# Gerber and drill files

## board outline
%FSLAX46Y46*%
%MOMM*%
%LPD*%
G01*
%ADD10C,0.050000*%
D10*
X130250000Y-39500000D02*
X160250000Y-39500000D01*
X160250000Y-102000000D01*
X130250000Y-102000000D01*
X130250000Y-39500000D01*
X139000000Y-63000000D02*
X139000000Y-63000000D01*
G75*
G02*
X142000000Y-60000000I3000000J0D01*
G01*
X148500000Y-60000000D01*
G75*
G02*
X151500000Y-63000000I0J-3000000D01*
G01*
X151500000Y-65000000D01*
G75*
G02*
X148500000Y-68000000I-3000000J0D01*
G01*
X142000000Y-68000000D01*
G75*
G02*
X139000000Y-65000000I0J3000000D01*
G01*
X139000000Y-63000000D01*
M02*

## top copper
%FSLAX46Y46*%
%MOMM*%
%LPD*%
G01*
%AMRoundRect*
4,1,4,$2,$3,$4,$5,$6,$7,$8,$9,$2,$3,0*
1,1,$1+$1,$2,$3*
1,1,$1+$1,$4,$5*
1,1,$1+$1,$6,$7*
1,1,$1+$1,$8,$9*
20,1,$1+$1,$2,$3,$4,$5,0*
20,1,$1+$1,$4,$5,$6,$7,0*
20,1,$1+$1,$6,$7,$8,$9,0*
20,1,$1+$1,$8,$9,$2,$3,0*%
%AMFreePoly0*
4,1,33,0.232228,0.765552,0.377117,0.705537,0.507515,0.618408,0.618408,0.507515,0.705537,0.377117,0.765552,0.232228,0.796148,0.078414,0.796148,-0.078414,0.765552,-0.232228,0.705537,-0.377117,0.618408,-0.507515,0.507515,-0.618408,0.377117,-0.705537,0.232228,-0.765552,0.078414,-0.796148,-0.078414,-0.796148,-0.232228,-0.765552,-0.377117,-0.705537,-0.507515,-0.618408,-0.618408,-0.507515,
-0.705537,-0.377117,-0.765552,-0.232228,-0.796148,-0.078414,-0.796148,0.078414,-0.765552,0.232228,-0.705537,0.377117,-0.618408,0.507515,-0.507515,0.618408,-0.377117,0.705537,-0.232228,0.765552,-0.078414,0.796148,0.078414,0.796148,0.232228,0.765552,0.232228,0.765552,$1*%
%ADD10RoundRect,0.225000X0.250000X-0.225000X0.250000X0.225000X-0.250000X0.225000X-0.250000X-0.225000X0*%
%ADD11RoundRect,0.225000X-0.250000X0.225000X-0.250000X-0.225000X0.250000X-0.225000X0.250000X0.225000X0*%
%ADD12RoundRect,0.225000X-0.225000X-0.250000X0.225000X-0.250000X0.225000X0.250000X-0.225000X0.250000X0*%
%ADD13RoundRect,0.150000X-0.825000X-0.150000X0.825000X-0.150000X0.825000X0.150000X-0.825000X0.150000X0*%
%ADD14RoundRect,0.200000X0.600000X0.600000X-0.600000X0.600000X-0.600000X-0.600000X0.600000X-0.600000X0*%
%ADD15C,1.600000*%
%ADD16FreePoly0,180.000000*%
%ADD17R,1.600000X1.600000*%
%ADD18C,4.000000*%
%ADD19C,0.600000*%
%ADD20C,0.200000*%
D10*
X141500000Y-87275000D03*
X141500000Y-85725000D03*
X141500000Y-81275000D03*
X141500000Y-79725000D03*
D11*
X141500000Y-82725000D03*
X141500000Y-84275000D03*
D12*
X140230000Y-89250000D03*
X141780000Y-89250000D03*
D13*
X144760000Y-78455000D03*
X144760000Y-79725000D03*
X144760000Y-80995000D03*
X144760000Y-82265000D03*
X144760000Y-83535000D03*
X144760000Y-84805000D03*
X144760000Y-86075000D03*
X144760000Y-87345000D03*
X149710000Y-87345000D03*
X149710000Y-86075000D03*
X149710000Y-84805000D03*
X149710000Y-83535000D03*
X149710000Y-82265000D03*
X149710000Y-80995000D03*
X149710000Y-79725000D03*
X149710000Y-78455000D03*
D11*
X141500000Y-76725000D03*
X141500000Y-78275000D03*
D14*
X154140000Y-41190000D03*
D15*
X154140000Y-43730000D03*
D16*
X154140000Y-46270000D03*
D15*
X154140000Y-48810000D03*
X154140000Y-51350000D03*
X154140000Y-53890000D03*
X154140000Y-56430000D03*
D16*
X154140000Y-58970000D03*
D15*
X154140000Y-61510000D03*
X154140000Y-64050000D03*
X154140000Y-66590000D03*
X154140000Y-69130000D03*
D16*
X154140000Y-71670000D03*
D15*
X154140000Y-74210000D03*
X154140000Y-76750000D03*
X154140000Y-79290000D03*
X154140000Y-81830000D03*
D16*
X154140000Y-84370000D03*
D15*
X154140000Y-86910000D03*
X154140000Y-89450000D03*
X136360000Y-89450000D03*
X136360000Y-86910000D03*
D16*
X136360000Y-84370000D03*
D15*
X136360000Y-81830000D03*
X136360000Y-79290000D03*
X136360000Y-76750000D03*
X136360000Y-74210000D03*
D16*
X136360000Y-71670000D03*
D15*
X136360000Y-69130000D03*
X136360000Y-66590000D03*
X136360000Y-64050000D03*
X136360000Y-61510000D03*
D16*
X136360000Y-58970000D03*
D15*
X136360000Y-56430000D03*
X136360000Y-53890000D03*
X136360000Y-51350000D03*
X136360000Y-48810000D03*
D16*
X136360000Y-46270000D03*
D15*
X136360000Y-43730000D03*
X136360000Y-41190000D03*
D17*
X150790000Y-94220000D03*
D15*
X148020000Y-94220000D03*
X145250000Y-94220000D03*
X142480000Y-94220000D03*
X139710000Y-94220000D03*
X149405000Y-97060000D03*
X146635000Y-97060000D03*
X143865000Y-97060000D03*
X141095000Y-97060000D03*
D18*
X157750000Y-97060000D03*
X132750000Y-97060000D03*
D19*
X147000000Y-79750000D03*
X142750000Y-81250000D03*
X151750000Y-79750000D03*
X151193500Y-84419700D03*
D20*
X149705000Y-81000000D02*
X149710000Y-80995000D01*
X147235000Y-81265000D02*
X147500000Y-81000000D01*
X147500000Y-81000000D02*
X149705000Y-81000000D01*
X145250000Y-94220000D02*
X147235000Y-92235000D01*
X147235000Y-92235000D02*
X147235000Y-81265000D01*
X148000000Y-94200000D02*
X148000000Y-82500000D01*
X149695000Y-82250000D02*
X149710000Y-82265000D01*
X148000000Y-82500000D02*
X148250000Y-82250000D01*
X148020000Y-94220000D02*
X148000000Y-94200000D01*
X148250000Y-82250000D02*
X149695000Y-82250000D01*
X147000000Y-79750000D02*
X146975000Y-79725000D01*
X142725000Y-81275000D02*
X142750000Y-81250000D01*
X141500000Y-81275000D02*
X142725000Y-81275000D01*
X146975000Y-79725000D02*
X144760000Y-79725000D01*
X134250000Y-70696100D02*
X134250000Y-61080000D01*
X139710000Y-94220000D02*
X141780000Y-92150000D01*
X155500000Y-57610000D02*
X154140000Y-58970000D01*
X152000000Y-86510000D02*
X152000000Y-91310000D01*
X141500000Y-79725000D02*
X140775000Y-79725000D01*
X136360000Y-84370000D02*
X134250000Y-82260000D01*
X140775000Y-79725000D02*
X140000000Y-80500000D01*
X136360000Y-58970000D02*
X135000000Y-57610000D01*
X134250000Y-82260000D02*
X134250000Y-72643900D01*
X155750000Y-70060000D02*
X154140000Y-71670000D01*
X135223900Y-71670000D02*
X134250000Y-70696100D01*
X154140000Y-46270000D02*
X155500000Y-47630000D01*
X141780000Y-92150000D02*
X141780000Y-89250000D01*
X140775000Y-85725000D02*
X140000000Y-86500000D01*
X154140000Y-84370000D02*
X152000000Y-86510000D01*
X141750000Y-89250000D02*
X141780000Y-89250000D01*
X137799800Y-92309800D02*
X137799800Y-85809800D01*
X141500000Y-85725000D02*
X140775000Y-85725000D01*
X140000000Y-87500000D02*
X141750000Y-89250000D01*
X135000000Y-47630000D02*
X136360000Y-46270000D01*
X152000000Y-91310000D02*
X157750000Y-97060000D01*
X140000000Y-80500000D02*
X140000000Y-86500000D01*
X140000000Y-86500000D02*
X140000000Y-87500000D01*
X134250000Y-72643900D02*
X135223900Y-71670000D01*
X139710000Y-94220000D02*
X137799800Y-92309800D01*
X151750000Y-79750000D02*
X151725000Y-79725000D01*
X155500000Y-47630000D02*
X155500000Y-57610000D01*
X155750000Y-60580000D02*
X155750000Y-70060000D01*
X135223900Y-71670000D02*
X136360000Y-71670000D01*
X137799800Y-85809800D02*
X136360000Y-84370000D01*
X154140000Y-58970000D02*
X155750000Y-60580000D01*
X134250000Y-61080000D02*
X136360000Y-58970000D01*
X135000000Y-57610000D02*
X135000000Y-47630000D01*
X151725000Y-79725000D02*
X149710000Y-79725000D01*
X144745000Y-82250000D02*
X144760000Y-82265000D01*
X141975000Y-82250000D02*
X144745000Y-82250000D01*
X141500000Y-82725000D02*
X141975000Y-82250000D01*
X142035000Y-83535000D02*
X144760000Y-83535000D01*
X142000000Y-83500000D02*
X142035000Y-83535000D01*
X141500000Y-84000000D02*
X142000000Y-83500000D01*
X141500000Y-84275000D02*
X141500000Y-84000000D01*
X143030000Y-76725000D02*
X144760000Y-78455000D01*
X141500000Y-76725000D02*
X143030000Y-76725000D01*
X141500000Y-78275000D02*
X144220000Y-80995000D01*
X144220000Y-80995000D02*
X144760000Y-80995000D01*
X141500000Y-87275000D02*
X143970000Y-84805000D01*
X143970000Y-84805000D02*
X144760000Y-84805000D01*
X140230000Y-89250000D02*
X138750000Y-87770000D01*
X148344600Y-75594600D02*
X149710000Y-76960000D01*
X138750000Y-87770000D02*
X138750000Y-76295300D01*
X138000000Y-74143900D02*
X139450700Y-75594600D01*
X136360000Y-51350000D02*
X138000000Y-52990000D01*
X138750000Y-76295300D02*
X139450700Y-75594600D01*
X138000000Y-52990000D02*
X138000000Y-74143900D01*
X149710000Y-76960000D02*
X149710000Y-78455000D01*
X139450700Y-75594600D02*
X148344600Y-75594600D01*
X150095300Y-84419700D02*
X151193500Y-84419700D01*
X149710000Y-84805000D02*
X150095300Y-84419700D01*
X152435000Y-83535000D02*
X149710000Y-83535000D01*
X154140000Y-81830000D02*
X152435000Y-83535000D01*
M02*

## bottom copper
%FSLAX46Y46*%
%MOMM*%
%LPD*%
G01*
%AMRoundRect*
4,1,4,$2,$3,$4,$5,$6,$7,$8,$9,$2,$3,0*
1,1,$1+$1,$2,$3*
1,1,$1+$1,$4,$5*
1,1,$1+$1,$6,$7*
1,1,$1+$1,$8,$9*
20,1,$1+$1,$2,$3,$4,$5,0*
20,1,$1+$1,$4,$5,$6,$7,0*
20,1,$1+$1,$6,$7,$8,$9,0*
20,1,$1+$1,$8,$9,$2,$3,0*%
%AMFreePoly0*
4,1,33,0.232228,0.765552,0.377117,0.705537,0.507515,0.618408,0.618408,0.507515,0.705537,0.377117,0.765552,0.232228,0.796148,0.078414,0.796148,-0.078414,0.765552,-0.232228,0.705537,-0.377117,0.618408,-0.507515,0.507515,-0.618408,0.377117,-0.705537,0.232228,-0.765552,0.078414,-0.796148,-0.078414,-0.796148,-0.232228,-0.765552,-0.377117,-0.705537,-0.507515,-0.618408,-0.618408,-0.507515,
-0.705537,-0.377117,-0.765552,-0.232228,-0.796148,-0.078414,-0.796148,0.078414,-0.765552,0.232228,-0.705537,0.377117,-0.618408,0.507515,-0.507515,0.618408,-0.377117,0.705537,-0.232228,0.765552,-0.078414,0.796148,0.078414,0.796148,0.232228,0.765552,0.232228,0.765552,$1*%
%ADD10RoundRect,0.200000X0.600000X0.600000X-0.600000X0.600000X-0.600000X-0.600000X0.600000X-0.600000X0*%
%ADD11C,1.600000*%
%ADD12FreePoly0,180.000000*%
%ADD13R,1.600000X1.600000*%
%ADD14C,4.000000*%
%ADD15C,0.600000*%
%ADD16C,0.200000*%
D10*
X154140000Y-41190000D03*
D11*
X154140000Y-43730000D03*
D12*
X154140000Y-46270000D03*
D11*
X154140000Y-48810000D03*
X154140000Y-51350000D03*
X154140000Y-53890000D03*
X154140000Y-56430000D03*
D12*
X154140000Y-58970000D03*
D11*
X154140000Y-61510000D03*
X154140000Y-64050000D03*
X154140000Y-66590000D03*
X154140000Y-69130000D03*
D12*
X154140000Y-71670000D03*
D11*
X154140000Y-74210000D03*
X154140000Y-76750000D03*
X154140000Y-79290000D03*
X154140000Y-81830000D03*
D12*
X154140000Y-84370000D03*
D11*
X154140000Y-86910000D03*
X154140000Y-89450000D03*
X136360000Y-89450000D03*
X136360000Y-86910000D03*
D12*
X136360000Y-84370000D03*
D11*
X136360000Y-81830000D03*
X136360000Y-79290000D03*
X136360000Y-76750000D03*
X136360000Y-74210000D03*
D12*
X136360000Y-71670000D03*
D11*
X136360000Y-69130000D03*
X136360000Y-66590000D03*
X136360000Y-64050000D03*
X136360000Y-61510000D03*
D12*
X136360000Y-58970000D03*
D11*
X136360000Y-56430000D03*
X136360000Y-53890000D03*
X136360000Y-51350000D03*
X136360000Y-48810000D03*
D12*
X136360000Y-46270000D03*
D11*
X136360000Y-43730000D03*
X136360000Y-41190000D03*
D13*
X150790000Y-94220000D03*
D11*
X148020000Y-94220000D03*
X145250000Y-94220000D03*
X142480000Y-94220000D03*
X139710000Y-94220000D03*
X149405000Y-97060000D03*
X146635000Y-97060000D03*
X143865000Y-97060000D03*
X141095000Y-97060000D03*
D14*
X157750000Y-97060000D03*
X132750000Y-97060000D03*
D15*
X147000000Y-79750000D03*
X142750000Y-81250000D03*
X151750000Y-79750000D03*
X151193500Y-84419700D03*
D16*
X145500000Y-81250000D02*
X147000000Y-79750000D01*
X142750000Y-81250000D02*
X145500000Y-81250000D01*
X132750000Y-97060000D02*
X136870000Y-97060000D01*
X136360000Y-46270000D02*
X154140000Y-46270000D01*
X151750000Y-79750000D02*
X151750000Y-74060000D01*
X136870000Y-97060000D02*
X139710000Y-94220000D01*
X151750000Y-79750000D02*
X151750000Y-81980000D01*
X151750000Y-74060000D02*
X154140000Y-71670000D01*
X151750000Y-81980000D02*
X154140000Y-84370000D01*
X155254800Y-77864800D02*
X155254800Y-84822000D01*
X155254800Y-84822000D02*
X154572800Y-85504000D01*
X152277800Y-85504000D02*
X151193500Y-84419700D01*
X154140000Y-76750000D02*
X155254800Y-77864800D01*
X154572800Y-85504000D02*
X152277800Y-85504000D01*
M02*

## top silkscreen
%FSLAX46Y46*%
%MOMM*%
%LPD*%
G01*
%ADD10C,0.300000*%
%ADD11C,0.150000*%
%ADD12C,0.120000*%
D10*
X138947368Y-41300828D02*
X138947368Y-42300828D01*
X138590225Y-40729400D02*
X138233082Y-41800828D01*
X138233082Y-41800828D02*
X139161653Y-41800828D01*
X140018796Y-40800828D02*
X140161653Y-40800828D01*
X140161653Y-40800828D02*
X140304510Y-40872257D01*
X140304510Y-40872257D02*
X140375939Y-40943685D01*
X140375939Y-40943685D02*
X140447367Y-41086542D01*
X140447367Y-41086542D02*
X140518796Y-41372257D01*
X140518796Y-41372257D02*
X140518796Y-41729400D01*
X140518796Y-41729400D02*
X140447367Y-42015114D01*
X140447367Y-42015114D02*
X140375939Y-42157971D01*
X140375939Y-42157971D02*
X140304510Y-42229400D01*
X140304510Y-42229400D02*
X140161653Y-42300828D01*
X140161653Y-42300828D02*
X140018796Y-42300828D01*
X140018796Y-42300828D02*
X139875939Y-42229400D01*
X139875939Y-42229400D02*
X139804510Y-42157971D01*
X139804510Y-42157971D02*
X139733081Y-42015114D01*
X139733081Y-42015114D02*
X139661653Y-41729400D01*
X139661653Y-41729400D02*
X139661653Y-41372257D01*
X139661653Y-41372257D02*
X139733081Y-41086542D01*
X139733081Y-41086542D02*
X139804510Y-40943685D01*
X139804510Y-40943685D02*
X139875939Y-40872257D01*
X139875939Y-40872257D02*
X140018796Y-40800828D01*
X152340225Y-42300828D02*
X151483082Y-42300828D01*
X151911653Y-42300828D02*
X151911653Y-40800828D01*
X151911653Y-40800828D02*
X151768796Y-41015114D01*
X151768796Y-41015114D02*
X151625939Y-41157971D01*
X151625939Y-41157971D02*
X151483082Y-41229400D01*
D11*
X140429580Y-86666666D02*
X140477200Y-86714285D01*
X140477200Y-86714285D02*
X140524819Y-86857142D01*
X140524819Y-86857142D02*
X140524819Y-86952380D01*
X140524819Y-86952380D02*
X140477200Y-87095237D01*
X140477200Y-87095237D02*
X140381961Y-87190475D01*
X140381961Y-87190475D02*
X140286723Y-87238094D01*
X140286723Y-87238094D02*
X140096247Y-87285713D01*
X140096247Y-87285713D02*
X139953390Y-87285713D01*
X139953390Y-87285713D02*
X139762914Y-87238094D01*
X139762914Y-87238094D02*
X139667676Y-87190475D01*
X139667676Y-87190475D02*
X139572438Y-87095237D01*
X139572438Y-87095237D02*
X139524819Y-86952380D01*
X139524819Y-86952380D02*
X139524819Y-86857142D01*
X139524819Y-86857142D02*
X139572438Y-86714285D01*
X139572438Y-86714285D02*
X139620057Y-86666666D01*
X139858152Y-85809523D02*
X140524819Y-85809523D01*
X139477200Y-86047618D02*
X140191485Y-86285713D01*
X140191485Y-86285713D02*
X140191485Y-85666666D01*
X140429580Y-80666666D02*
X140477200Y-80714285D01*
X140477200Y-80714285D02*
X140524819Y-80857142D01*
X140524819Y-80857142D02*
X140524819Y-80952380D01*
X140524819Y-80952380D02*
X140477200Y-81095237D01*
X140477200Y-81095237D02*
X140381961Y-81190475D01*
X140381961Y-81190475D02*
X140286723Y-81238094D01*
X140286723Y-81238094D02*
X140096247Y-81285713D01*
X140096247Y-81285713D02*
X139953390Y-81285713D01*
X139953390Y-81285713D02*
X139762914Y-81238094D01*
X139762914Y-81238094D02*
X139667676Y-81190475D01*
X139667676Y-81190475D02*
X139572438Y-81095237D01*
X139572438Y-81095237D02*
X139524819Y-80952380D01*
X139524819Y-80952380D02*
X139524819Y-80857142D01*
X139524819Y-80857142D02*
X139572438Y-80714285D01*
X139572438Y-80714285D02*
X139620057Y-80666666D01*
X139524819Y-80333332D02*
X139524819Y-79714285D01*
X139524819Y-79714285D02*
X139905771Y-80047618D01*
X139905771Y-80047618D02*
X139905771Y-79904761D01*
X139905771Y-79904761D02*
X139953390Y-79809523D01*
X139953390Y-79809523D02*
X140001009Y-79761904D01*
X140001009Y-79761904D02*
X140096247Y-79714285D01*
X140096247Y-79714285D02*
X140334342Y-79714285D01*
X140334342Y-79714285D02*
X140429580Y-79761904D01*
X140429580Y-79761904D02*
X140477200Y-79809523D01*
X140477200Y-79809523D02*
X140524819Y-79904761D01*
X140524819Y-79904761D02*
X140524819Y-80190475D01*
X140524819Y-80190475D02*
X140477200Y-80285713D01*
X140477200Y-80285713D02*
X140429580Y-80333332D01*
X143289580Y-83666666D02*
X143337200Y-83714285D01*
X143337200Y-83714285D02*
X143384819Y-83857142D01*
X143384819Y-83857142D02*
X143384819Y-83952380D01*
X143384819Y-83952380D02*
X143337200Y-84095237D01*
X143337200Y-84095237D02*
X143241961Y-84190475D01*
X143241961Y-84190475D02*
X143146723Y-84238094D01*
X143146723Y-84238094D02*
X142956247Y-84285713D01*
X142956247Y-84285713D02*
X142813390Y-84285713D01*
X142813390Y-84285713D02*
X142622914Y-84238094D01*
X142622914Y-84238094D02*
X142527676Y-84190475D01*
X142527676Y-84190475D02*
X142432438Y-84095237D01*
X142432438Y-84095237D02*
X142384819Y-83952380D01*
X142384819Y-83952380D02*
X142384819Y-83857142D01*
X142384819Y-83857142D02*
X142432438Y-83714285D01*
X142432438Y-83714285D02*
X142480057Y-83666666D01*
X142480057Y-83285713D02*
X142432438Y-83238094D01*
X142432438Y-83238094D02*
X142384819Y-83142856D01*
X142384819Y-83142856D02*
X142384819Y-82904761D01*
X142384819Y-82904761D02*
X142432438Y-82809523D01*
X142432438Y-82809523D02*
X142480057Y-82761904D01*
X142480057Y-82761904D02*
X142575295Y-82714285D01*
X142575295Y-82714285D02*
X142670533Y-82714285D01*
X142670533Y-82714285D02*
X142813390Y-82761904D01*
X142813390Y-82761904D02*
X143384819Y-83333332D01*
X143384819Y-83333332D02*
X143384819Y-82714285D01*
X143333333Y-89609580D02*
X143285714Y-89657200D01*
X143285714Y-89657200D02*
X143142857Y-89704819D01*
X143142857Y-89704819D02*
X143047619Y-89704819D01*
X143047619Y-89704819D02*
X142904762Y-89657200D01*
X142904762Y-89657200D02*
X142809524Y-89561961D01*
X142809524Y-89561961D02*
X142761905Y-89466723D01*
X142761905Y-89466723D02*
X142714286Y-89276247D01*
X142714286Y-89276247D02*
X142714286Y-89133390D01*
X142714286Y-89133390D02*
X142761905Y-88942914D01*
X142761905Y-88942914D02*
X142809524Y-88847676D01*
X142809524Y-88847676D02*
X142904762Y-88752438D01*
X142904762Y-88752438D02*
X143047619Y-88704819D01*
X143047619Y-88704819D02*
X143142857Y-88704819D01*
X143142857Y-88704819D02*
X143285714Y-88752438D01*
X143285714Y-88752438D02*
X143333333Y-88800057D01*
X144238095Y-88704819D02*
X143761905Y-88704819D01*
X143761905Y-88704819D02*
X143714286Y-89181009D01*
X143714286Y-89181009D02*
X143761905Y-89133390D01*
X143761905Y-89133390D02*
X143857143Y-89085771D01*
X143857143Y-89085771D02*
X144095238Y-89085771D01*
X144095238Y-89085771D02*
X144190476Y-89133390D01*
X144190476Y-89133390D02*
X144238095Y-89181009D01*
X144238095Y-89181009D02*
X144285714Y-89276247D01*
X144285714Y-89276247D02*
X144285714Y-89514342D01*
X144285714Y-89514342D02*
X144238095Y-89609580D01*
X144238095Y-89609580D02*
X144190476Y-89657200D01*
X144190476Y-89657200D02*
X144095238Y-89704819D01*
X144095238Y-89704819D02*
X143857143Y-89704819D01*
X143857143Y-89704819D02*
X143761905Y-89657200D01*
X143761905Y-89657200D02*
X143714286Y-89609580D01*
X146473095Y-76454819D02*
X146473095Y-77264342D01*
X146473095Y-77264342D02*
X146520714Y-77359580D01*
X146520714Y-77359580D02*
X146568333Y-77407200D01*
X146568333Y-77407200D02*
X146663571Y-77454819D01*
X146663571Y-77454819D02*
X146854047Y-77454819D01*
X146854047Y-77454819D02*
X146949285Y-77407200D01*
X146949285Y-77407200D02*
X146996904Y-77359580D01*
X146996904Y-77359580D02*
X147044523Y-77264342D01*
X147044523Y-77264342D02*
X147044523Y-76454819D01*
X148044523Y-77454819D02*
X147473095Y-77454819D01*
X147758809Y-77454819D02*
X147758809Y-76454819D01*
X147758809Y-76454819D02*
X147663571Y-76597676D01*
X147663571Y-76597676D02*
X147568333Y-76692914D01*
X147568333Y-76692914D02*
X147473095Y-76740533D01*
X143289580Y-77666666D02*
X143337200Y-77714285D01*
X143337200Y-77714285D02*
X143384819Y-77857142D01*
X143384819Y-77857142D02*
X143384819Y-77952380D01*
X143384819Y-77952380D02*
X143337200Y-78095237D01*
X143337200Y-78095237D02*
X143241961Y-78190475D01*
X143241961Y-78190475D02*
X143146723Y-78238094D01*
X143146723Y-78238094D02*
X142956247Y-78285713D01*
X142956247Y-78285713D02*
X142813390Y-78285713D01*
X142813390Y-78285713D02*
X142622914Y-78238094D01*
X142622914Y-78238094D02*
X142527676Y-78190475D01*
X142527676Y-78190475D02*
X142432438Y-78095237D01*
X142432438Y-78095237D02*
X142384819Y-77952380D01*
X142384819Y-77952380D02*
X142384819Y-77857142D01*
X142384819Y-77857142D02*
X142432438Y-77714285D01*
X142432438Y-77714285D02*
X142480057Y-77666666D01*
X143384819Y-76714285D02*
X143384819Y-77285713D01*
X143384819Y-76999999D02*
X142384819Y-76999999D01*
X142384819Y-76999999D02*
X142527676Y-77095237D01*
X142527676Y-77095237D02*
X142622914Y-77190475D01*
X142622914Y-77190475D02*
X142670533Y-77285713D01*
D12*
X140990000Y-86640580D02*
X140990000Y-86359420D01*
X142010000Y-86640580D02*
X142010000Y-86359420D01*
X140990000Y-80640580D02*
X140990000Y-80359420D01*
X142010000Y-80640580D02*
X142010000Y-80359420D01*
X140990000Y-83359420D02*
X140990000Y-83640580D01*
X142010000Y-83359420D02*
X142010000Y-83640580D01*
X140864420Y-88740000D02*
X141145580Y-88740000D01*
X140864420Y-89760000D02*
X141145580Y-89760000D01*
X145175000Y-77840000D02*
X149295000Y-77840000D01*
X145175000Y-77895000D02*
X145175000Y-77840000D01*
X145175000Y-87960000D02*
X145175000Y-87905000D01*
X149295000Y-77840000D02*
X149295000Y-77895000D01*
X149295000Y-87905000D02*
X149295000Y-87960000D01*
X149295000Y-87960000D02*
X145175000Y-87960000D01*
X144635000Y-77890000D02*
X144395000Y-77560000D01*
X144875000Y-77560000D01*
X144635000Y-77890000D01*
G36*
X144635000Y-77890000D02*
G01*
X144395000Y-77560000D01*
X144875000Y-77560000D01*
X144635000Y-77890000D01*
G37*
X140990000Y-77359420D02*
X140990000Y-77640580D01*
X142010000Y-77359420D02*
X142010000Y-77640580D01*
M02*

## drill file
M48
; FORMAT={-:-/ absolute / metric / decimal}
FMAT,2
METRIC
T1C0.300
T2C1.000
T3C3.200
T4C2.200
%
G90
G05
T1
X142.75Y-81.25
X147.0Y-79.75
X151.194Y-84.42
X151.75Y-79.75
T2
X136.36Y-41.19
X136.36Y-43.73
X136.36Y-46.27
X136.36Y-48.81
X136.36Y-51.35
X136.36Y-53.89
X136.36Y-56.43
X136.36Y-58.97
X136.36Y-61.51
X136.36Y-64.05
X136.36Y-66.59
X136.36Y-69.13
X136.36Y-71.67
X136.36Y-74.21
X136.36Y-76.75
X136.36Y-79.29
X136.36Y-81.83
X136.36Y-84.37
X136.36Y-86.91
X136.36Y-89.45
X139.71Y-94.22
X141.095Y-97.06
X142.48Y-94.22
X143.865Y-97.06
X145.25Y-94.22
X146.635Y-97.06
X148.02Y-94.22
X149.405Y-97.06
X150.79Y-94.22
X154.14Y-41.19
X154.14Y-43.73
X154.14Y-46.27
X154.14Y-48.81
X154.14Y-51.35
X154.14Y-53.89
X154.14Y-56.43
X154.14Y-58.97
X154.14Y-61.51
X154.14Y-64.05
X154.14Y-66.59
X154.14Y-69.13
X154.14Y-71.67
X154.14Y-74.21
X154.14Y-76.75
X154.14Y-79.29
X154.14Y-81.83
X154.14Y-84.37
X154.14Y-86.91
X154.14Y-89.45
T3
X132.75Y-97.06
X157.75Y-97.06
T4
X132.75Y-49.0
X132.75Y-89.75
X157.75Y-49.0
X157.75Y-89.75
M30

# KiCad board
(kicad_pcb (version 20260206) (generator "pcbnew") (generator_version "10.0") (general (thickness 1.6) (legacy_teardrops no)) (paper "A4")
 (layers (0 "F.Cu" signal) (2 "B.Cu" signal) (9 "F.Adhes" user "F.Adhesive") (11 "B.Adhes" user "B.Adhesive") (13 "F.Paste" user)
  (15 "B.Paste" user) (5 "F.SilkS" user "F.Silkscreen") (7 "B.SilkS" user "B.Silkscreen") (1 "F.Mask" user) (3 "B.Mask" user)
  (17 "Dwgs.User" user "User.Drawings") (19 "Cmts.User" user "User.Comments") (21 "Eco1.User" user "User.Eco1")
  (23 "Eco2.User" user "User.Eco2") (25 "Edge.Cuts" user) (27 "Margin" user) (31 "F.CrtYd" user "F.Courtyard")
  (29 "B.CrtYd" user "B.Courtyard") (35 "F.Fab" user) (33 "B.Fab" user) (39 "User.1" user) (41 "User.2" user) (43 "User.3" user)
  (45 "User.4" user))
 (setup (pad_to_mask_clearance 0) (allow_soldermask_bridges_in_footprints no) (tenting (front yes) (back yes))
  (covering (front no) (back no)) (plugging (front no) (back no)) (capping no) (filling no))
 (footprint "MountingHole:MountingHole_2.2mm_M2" (layer "F.Cu") (at 132.75 49)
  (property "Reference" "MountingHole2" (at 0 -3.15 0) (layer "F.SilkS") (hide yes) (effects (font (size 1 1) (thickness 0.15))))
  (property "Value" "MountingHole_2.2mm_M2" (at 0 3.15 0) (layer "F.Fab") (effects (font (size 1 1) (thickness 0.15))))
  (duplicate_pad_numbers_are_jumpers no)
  (pad "" np_thru_hole circle (at 0 0) (size 2.2 2.2) (drill 2.2) (layers "*.Cu" "*.Mask")))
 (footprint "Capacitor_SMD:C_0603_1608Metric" (layer "F.Cu") (at 141.5 86.5 90)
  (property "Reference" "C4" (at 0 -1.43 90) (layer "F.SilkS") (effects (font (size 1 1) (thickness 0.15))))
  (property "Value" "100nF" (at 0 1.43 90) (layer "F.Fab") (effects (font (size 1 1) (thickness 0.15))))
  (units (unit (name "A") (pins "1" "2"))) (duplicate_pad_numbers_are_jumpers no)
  (fp_line (start -0.14058 -0.51) (end 0.14058 -0.51) (stroke (width 0.12) (type solid)) (layer "F.SilkS"))
  (fp_line (start -0.14058 0.51) (end 0.14058 0.51) (stroke (width 0.12) (type solid)) (layer "F.SilkS"))
  (pad "1" smd roundrect (at -0.775 0 90) (size 0.9 0.95) (layers "F.Cu" "F.Mask" "F.Paste") (roundrect_rratio 0.25) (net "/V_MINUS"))
  (pad "2" smd roundrect (at 0.775 0 90) (size 0.9 0.95) (layers "F.Cu" "F.Mask" "F.Paste") (roundrect_rratio 0.25) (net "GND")))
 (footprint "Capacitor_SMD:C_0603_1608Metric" (layer "F.Cu") (at 141.5 80.5 90)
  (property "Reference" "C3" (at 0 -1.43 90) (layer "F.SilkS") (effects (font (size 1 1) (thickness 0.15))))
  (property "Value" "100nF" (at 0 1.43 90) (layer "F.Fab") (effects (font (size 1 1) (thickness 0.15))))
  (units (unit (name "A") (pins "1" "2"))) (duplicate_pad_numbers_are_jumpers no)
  (fp_line (start -0.14058 -0.51) (end 0.14058 -0.51) (stroke (width 0.12) (type solid)) (layer "F.SilkS"))
  (fp_line (start -0.14058 0.51) (end 0.14058 0.51) (stroke (width 0.12) (type solid)) (layer "F.SilkS"))
  (pad "1" smd roundrect (at -0.775 0 90) (size 0.9 0.95) (layers "F.Cu" "F.Mask" "F.Paste") (roundrect_rratio 0.25) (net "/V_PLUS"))
  (pad "2" smd roundrect (at 0.775 0 90) (size 0.9 0.95) (layers "F.Cu" "F.Mask" "F.Paste") (roundrect_rratio 0.25) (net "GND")))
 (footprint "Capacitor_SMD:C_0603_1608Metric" (layer "F.Cu") (at 141.5 83.5 -90)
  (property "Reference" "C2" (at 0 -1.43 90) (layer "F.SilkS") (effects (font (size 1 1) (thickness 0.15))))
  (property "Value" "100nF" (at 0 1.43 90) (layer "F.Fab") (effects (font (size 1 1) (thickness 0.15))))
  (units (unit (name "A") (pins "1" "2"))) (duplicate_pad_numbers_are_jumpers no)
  (fp_line (start -0.14058 0.51) (end 0.14058 0.51) (stroke (width 0.12) (type solid)) (layer "F.SilkS"))
  (fp_line (start -0.14058 -0.51) (end 0.14058 -0.51) (stroke (width 0.12) (type solid)) (layer "F.SilkS"))
  (pad "1" smd roundrect (at -0.775 0 270) (size 0.9 0.95) (layers "F.Cu" "F.Mask" "F.Paste") (roundrect_rratio 0.25) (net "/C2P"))
  (pad "2" smd roundrect (at 0.775 0 270) (size 0.9 0.95) (layers "F.Cu" "F.Mask" "F.Paste") (roundrect_rratio 0.25) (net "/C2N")))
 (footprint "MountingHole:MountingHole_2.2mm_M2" (layer "F.Cu") (at 132.75 89.75)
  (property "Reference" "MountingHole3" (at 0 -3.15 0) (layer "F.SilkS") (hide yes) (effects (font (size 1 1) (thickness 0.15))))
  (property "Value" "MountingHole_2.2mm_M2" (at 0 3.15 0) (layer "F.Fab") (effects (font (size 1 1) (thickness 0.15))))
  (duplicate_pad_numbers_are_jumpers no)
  (pad "" np_thru_hole circle (at 0 0) (size 2.2 2.2) (drill 2.2) (layers "*.Cu" "*.Mask")))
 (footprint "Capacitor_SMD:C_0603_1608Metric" (layer "F.Cu") (at 141.005 89.25)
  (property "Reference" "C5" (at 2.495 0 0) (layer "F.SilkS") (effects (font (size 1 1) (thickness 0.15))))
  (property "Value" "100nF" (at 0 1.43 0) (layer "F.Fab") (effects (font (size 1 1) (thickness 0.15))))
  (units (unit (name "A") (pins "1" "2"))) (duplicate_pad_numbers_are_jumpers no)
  (fp_line (start -0.14058 -0.51) (end 0.14058 -0.51) (stroke (width 0.12) (type solid)) (layer "F.SilkS"))
  (fp_line (start -0.14058 0.51) (end 0.14058 0.51) (stroke (width 0.12) (type solid)) (layer "F.SilkS"))
  (pad "1" smd roundrect (at -0.775 0) (size 0.9 0.95) (layers "F.Cu" "F.Mask" "F.Paste") (roundrect_rratio 0.25) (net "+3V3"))
  (pad "2" smd roundrect (at 0.775 0) (size 0.9 0.95) (layers "F.Cu" "F.Mask" "F.Paste") (roundrect_rratio 0.25) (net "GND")))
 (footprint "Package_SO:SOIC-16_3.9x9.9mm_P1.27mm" (layer "F.Cu") (at 147.235 82.9)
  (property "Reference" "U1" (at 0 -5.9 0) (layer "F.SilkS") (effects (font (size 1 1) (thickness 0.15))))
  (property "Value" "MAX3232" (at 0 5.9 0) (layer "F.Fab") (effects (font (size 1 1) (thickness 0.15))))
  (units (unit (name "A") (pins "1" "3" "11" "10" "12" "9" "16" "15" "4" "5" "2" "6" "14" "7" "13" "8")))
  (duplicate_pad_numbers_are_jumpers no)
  (fp_line (start -2.06 -5.06) (end 2.06 -5.06) (stroke (width 0.12) (type solid)) (layer "F.SilkS"))
  (fp_line (start -2.06 -5.005) (end -2.06 -5.06) (stroke (width 0.12) (type solid)) (layer "F.SilkS"))
  (fp_line (start -2.06 5.06) (end -2.06 5.005) (stroke (width 0.12) (type solid)) (layer "F.SilkS"))
  (fp_line (start 2.06 -5.06) (end 2.06 -5.005) (stroke (width 0.12) (type solid)) (layer "F.SilkS"))
  (fp_line (start 2.06 5.005) (end 2.06 5.06) (stroke (width 0.12) (type solid)) (layer "F.SilkS"))
  (fp_line (start 2.06 5.06) (end -2.06 5.06) (stroke (width 0.12) (type solid)) (layer "F.SilkS"))
  (fp_poly (pts (xy -2.6 -5.01) (xy -2.84 -5.34) (xy -2.36 -5.34)) (stroke (width 0.12) (type solid)) (fill yes) (layer "F.SilkS"))
  (pad "1" smd roundrect (at -2.475 -4.445) (size 1.95 0.6) (layers "F.Cu" "F.Mask" "F.Paste") (roundrect_rratio 0.25) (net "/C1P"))
  (pad "2" smd roundrect (at -2.475 -3.175) (size 1.95 0.6) (layers "F.Cu" "F.Mask" "F.Paste") (roundrect_rratio 0.25) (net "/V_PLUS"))
  (pad "3" smd roundrect (at -2.475 -1.905) (size 1.95 0.6) (layers "F.Cu" "F.Mask" "F.Paste") (roundrect_rratio 0.25) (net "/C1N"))
  (pad "4" smd roundrect (at -2.475 -0.635) (size 1.95 0.6) (layers "F.Cu" "F.Mask" "F.Paste") (roundrect_rratio 0.25) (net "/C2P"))
  (pad "5" smd roundrect (at -2.475 0.635) (size 1.95 0.6) (layers "F.Cu" "F.Mask" "F.Paste") (roundrect_rratio 0.25) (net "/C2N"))
  (pad "6" smd roundrect (at -2.475 1.905) (size 1.95 0.6) (layers "F.Cu" "F.Mask" "F.Paste") (roundrect_rratio 0.25) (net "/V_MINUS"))
  (pad "7" smd roundrect (at -2.475 3.175) (size 1.95 0.6) (layers "F.Cu" "F.Mask" "F.Paste") (roundrect_rratio 0.25)
   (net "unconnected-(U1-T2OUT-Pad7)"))
  (pad "8" smd roundrect (at -2.475 4.445) (size 1.95 0.6) (layers "F.Cu" "F.Mask" "F.Paste") (roundrect_rratio 0.25)
   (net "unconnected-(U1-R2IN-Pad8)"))
  (pad "9" smd roundrect (at 2.475 4.445) (size 1.95 0.6) (layers "F.Cu" "F.Mask" "F.Paste") (roundrect_rratio 0.25)
   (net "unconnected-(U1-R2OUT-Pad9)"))
  (pad "10" smd roundrect (at 2.475 3.175) (size 1.95 0.6) (layers "F.Cu" "F.Mask" "F.Paste") (roundrect_rratio 0.25)
   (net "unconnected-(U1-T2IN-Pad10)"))
  (pad "11" smd roundrect (at 2.475 1.905) (size 1.95 0.6) (layers "F.Cu" "F.Mask" "F.Paste") (roundrect_rratio 0.25) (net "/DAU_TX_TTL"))
  (pad "12" smd roundrect (at 2.475 0.635) (size 1.95 0.6) (layers "F.Cu" "F.Mask" "F.Paste") (roundrect_rratio 0.25) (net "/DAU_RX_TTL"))
  (pad "13" smd roundrect (at 2.475 -0.635) (size 1.95 0.6) (layers "F.Cu" "F.Mask" "F.Paste") (roundrect_rratio 0.25) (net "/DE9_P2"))
  (pad "14" smd roundrect (at 2.475 -1.905) (size 1.95 0.6) (layers "F.Cu" "F.Mask" "F.Paste") (roundrect_rratio 0.25) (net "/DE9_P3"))
  (pad "15" smd roundrect (at 2.475 -3.175) (size 1.95 0.6) (layers "F.Cu" "F.Mask" "F.Paste") (roundrect_rratio 0.25) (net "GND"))
  (pad "16" smd roundrect (at 2.475 -4.445) (size 1.95 0.6) (layers "F.Cu" "F.Mask" "F.Paste") (roundrect_rratio 0.25) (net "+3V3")))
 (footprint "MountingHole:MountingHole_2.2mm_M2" (layer "F.Cu") (at 157.75 49)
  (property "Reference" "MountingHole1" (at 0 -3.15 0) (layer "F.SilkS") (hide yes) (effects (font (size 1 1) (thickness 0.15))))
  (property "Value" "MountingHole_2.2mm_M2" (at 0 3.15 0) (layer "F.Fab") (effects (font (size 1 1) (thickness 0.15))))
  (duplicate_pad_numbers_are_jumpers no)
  (pad "" np_thru_hole circle (at 0 0) (size 2.2 2.2) (drill 2.2) (layers "*.Cu" "*.Mask")))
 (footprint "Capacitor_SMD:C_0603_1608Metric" (layer "F.Cu") (at 141.5 77.5 -90)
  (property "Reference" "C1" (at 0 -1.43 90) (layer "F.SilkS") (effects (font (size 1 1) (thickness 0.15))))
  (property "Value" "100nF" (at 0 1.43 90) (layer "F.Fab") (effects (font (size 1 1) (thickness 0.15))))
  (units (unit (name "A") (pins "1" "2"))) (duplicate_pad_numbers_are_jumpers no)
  (fp_line (start -0.14058 0.51) (end 0.14058 0.51) (stroke (width 0.12) (type solid)) (layer "F.SilkS"))
  (fp_line (start -0.14058 -0.51) (end 0.14058 -0.51) (stroke (width 0.12) (type solid)) (layer "F.SilkS"))
  (pad "1" smd roundrect (at -0.775 0 270) (size 0.9 0.95) (layers "F.Cu" "F.Mask" "F.Paste") (roundrect_rratio 0.25) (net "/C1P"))
  (pad "2" smd roundrect (at 0.775 0 270) (size 0.9 0.95) (layers "F.Cu" "F.Mask" "F.Paste") (roundrect_rratio 0.25) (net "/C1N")))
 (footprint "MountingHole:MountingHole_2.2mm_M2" (layer "F.Cu") (at 157.75 89.75)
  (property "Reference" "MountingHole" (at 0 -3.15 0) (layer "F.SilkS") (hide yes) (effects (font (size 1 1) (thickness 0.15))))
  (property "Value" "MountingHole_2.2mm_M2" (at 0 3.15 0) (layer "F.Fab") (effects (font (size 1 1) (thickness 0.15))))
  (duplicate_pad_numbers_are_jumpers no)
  (pad "" np_thru_hole circle (at 0 0) (size 2.2 2.2) (drill 2.2) (layers "*.Cu" "*.Mask")))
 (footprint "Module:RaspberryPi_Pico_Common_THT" (layer "B.Cu") (at 154.14 41.19 180)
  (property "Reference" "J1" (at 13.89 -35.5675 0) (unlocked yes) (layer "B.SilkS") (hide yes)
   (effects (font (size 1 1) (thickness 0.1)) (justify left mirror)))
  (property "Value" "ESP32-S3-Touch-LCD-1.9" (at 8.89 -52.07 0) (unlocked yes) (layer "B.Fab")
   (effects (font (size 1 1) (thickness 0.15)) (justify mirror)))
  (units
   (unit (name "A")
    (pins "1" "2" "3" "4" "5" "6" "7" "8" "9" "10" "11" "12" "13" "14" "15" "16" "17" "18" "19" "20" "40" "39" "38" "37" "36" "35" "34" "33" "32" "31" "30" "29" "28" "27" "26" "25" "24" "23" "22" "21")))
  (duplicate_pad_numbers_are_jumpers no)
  (pad "1" thru_hole roundrect (at 0 0 180) (size 1.6 1.6) (drill 1) (layers "*.Cu" "*.Mask") (remove_unused_layers no)
   (roundrect_rratio 0.125) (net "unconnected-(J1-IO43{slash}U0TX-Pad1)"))
  (pad "2" thru_hole circle (at 0 -2.54 180) (size 1.6 1.6) (drill 1) (layers "*.Cu" "*.Mask") (remove_unused_layers no)
   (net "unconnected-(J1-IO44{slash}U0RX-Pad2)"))
  (pad "3" thru_hole custom (at 0 -5.08 180) (size 1.6 1.6) (drill 1) (layers "*.Cu" "*.Mask") (remove_unused_layers no) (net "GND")
   (options (clearance outline) (anchor circle)) (primitives))
  (pad "4" thru_hole circle (at 0 -7.62 180) (size 1.6 1.6) (drill 1) (layers "*.Cu" "*.Mask") (remove_unused_layers no)
   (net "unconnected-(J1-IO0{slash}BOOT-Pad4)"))
  (pad "5" thru_hole circle (at 0 -10.16 180) (size 1.6 1.6) (drill 1) (layers "*.Cu" "*.Mask") (remove_unused_layers no)
   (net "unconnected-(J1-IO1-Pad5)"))
  (pad "6" thru_hole circle (at 0 -12.7 180) (size 1.6 1.6) (drill 1) (layers "*.Cu" "*.Mask") (remove_unused_layers no)
   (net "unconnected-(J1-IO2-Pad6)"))
  (pad "7" thru_hole circle (at 0 -15.24 180) (size 1.6 1.6) (drill 1) (layers "*.Cu" "*.Mask") (remove_unused_layers no)
   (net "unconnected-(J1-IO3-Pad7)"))
  (pad "8" thru_hole custom (at 0 -17.78 180) (size 1.6 1.6) (drill 1) (layers "*.Cu" "*.Mask") (remove_unused_layers no) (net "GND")
   (options (clearance outline) (anchor circle)) (primitives))
  (pad "9" thru_hole circle (at 0 -20.32 180) (size 1.6 1.6) (drill 1) (layers "*.Cu" "*.Mask") (remove_unused_layers no)
   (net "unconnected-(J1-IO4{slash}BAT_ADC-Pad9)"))
  (pad "10" thru_hole circle (at 0 -22.86 180) (size 1.6 1.6) (drill 1) (layers "*.Cu" "*.Mask") (remove_unused_layers no)
   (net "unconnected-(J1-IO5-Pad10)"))
  (pad "11" thru_hole circle (at 0 -25.4 180) (size 1.6 1.6) (drill 1) (layers "*.Cu" "*.Mask") (remove_unused_layers no)
   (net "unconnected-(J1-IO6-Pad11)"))
  (pad "12" thru_hole circle (at 0 -27.94 180) (size 1.6 1.6) (drill 1) (layers "*.Cu" "*.Mask") (remove_unused_layers no)
   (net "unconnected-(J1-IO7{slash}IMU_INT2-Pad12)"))
  (pad "13" thru_hole custom (at 0 -30.48 180) (size 1.6 1.6) (drill 1) (layers "*.Cu" "*.Mask") (remove_unused_layers no) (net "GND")
   (options (clearance outline) (anchor circle)) (primitives))
  (pad "14" thru_hole circle (at 0 -33.02 180) (size 1.6 1.6) (drill 1) (layers "*.Cu" "*.Mask") (remove_unused_layers no)
   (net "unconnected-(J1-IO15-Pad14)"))
  (pad "15" thru_hole circle (at 0 -35.56 180) (size 1.6 1.6) (drill 1) (layers "*.Cu" "*.Mask") (remove_unused_layers no)
   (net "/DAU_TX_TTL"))
  (pad "16" thru_hole circle (at 0 -38.1 180) (size 1.6 1.6) (drill 1) (layers "*.Cu" "*.Mask") (remove_unused_layers no)
   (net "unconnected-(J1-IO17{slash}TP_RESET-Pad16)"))
  (pad "17" thru_hole circle (at 0 -40.64 180) (size 1.6 1.6) (drill 1) (layers "*.Cu" "*.Mask") (remove_unused_layers no)
   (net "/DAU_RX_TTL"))
  (pad "18" thru_hole custom (at 0 -43.18 180) (size 1.6 1.6) (drill 1) (layers "*.Cu" "*.Mask") (remove_unused_layers no) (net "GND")
   (options (clearance outline) (anchor circle)) (primitives))
  (pad "19" thru_hole circle (at 0 -45.72 180) (size 1.6 1.6) (drill 1) (layers "*.Cu" "*.Mask") (remove_unused_layers no)
   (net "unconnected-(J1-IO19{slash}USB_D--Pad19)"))
  (pad "20" thru_hole circle (at 0 -48.26 180) (size 1.6 1.6) (drill 1) (layers "*.Cu" "*.Mask") (remove_unused_layers no)
   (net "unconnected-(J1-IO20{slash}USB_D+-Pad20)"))
  (pad "21" thru_hole circle (at 17.78 -48.26 180) (size 1.6 1.6) (drill 1) (layers "*.Cu" "*.Mask") (remove_unused_layers no)
   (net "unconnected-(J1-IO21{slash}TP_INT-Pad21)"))
  (pad "22" thru_hole circle (at 17.78 -45.72 180) (size 1.6 1.6) (drill 1) (layers "*.Cu" "*.Mask") (remove_unused_layers no)
   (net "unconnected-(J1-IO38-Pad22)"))
  (pad "23" thru_hole custom (at 17.78 -43.18 180) (size 1.6 1.6) (drill 1) (layers "*.Cu" "*.Mask") (remove_unused_layers no) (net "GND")
   (options (clearance outline) (anchor circle)) (primitives))
  (pad "24" thru_hole circle (at 17.78 -40.64 180) (size 1.6 1.6) (drill 1) (layers "*.Cu" "*.Mask") (remove_unused_layers no)
   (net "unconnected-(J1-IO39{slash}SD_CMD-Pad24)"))
  (pad "25" thru_hole circle (at 17.78 -38.1 180) (size 1.6 1.6) (drill 1) (layers "*.Cu" "*.Mask") (remove_unused_layers no)
   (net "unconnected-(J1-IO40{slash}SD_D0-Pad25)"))
  (pad "26" thru_hole circle (at 17.78 -35.56 180) (size 1.6 1.6) (drill 1) (layers "*.Cu" "*.Mask") (remove_unused_layers no)
   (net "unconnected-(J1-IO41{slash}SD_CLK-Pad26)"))
  (pad "27" thru_hole circle (at 17.78 -33.02 180) (size 1.6 1.6) (drill 1) (layers "*.Cu" "*.Mask") (remove_unused_layers no)
   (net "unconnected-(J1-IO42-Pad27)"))
  (pad "28" thru_hole custom (at 17.78 -30.48 180) (size 1.6 1.6) (drill 1) (layers "*.Cu" "*.Mask") (remove_unused_layers no) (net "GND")
   (options (clearance outline) (anchor circle)) (primitives))
  (pad "29" thru_hole circle (at 17.78 -27.94 180) (size 1.6 1.6) (drill 1) (layers "*.Cu" "*.Mask") (remove_unused_layers no)
   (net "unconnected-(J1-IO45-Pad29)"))
  (pad "30" thru_hole circle (at 17.78 -25.4 180) (size 1.6 1.6) (drill 1) (layers "*.Cu" "*.Mask") (remove_unused_layers no)
   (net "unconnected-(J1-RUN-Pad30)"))
  (pad "31" thru_hole circle (at 17.78 -22.86 180) (size 1.6 1.6) (drill 1) (layers "*.Cu" "*.Mask") (remove_unused_layers no)
   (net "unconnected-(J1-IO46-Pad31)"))
  (pad "32" thru_hole circle (at 17.78 -20.32 180) (size 1.6 1.6) (drill 1) (layers "*.Cu" "*.Mask") (remove_unused_layers no)
   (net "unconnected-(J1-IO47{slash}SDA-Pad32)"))
  (pad "33" thru_hole custom (at 17.78 -17.78 180) (size 1.6 1.6) (drill 1) (layers "*.Cu" "*.Mask") (remove_unused_layers no) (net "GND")
   (options (clearance outline) (anchor circle)) (primitives))
  (pad "34" thru_hole circle (at 17.78 -15.24 180) (size 1.6 1.6) (drill 1) (layers "*.Cu" "*.Mask") (remove_unused_layers no)
   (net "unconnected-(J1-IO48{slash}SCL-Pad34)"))
  (pad "35" thru_hole circle (at 17.78 -12.7 180) (size 1.6 1.6) (drill 1) (layers "*.Cu" "*.Mask") (remove_unused_layers no)
   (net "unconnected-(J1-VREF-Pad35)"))
  (pad "36" thru_hole circle (at 17.78 -10.16 180) (size 1.6 1.6) (drill 1) (layers "*.Cu" "*.Mask") (remove_unused_layers no) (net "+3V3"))
  (pad "37" thru_hole circle (at 17.78 -7.62 180) (size 1.6 1.6) (drill 1) (layers "*.Cu" "*.Mask") (remove_unused_layers no)
   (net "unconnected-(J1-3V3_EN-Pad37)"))
  (pad "38" thru_hole custom (at 17.78 -5.08 180) (size 1.6 1.6) (drill 1) (layers "*.Cu" "*.Mask") (remove_unused_layers no) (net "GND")
   (options (clearance outline) (anchor circle)) (primitives))
  (pad "39" thru_hole circle (at 17.78 -2.54 180) (size 1.6 1.6) (drill 1) (layers "*.Cu" "*.Mask") (remove_unused_layers no)
   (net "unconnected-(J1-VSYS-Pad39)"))
  (pad "40" thru_hole circle (at 17.78 0 180) (size 1.6 1.6) (drill 1) (layers "*.Cu" "*.Mask") (remove_unused_layers no)
   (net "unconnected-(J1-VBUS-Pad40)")))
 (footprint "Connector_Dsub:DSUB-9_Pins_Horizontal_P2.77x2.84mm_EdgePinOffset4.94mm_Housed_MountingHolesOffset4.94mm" (layer "B.Cu")
  (at 150.79 94.22 180)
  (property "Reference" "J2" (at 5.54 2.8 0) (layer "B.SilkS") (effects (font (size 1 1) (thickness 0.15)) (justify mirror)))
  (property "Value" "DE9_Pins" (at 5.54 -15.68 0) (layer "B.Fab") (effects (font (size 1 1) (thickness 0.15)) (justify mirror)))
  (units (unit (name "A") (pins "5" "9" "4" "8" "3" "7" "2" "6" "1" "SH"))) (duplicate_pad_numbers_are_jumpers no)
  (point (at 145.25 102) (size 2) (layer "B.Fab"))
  (pad "1" thru_hole rect (at 0 0 180) (size 1.6 1.6) (drill 1) (layers "*.Cu" "*.Mask") (remove_unused_layers no)
   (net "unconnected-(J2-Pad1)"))
  (pad "2" thru_hole circle (at 2.77 0 180) (size 1.6 1.6) (drill 1) (layers "*.Cu" "*.Mask") (remove_unused_layers no) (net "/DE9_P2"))
  (pad "3" thru_hole circle (at 5.54 0 180) (size 1.6 1.6) (drill 1) (layers "*.Cu" "*.Mask") (remove_unused_layers no) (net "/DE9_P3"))
  (pad "4" thru_hole circle (at 8.31 0 180) (size 1.6 1.6) (drill 1) (layers "*.Cu" "*.Mask") (remove_unused_layers no)
   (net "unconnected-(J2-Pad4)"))
  (pad "5" thru_hole circle (at 11.08 0 180) (size 1.6 1.6) (drill 1) (layers "*.Cu" "*.Mask") (remove_unused_layers no) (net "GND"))
  (pad "6" thru_hole circle (at 1.385 -2.84 180) (size 1.6 1.6) (drill 1) (layers "*.Cu" "*.Mask") (remove_unused_layers no)
   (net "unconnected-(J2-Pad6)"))
  (pad "7" thru_hole circle (at 4.155 -2.84 180) (size 1.6 1.6) (drill 1) (layers "*.Cu" "*.Mask") (remove_unused_layers no)
   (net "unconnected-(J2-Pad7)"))
  (pad "8" thru_hole circle (at 6.925 -2.84 180) (size 1.6 1.6) (drill 1) (layers "*.Cu" "*.Mask") (remove_unused_layers no)
   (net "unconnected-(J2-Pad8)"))
  (pad "9" thru_hole circle (at 9.695 -2.84 180) (size 1.6 1.6) (drill 1) (layers "*.Cu" "*.Mask") (remove_unused_layers no)
   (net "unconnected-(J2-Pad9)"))
  (pad "SH" thru_hole circle (at -6.96 -2.84 180) (size 4 4) (drill 3.2) (layers "*.Cu" "*.Mask") (remove_unused_layers no) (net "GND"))
  (pad "SH" thru_hole circle (at 18.04 -2.84 180) (size 4 4) (drill 3.2) (layers "*.Cu" "*.Mask") (remove_unused_layers no) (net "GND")))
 (gr_rect (start 130.25 39.5) (end 160.25 102) (stroke (width 0.05) (type default)) (fill no) (layer "Edge.Cuts"))
 (gr_rect (start 139 60) (end 151.5 68) (radius 3) (stroke (width 0.05) (type solid)) (fill no) (layer "Edge.Cuts"))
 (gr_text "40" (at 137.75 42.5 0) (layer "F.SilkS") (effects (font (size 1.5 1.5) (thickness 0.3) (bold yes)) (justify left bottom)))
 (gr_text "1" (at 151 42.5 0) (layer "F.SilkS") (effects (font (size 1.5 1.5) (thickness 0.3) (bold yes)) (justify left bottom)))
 (segment (start 149.705 81) (end 149.71 80.995) (width 0.2) (layer "F.Cu") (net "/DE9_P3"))
 (segment (start 147.235 81.265) (end 147.5 81) (width 0.2) (layer "F.Cu") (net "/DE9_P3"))
 (segment (start 147.5 81) (end 149.705 81) (width 0.2) (layer "F.Cu") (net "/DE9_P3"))
 (segment (start 145.25 94.22) (end 147.235 92.235) (width 0.2) (layer "F.Cu") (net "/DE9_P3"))
 (segment (start 147.235 92.235) (end 147.235 81.265) (width 0.2) (layer "F.Cu") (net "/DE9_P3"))
 (segment (start 148 94.2) (end 148 82.5) (width 0.2) (layer "F.Cu") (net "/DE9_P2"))
 (segment (start 149.695 82.25) (end 149.71 82.265) (width 0.2) (layer "F.Cu") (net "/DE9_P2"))
 (segment (start 148 82.5) (end 148.25 82.25) (width 0.2) (layer "F.Cu") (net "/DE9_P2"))
 (segment (start 148.02 94.22) (end 148 94.2) (width 0.2) (layer "F.Cu") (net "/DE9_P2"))
 (segment (start 148.25 82.25) (end 149.695 82.25) (width 0.2) (layer "F.Cu") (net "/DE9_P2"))
 (segment (start 147 79.75) (end 146.975 79.725) (width 0.2) (layer "F.Cu") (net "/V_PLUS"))
 (segment (start 142.725 81.275) (end 142.75 81.25) (width 0.2) (layer "F.Cu") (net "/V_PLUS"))
 (segment (start 141.5 81.275) (end 142.725 81.275) (width 0.2) (layer "F.Cu") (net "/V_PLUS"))
 (segment (start 146.975 79.725) (end 144.76 79.725) (width 0.2) (layer "F.Cu") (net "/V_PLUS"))
 (via (at 147 79.75) (size 0.6) (drill 0.3) (layers "F.Cu" "B.Cu") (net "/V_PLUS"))
 (via (at 142.75 81.25) (size 0.6) (drill 0.3) (layers "F.Cu" "B.Cu") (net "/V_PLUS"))
 (segment (start 145.5 81.25) (end 147 79.75) (width 0.2) (layer "B.Cu") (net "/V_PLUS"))
 (segment (start 142.75 81.25) (end 145.5 81.25) (width 0.2) (layer "B.Cu") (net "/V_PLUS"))
 (segment (start 134.25 70.6961) (end 134.25 61.08) (width 0.2) (layer "F.Cu") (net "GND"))
 (segment (start 139.71 94.22) (end 141.78 92.15) (width 0.2) (layer "F.Cu") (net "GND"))
 (segment (start 155.5 57.61) (end 154.14 58.97) (width 0.2) (layer "F.Cu") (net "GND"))
 (segment (start 152 86.51) (end 152 91.31) (width 0.2) (layer "F.Cu") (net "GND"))
 (segment (start 141.5 79.725) (end 140.775 79.725) (width 0.2) (layer "F.Cu") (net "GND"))
 (segment (start 136.36 84.37) (end 134.25 82.26) (width 0.2) (layer "F.Cu") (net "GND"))
 (segment (start 140.775 79.725) (end 140 80.5) (width 0.2) (layer "F.Cu") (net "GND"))
 (segment (start 136.36 58.97) (end 135 57.61) (width 0.2) (layer "F.Cu") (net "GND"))
 (segment (start 134.25 82.26) (end 134.25 72.6439) (width 0.2) (layer "F.Cu") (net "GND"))
 (segment (start 155.75 70.06) (end 154.14 71.67) (width 0.2) (layer "F.Cu") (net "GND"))
 (segment (start 135.2239 71.67) (end 134.25 70.6961) (width 0.2) (layer "F.Cu") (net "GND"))
 (segment (start 154.14 46.27) (end 155.5 47.63) (width 0.2) (layer "F.Cu") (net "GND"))
 (segment (start 141.78 92.15) (end 141.78 89.25) (width 0.2) (layer "F.Cu") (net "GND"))
 (segment (start 140.775 85.725) (end 140 86.5) (width 0.2) (layer "F.Cu") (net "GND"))
 (segment (start 154.14 84.37) (end 152 86.51) (width 0.2) (layer "F.Cu") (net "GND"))
 (segment (start 141.75 89.25) (end 141.78 89.25) (width 0.2) (layer "F.Cu") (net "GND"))
 (segment (start 137.7998 92.3098) (end 137.7998 85.8098) (width 0.2) (layer "F.Cu") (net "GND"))
 (segment (start 141.5 85.725) (end 140.775 85.725) (width 0.2) (layer "F.Cu") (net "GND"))
 (segment (start 140 87.5) (end 141.75 89.25) (width 0.2) (layer "F.Cu") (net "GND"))
 (segment (start 135 47.63) (end 136.36 46.27) (width 0.2) (layer "F.Cu") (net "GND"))
 (segment (start 152 91.31) (end 157.75 97.06) (width 0.2) (layer "F.Cu") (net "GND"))
 (segment (start 140 80.5) (end 140 86.5) (width 0.2) (layer "F.Cu") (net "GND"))
 (segment (start 140 86.5) (end 140 87.5) (width 0.2) (layer "F.Cu") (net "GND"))
 (segment (start 134.25 72.6439) (end 135.2239 71.67) (width 0.2) (layer "F.Cu") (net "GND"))
 (segment (start 139.71 94.22) (end 137.7998 92.3098) (width 0.2) (layer "F.Cu") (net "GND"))
 (segment (start 151.75 79.75) (end 151.725 79.725) (width 0.2) (layer "F.Cu") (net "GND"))
 (segment (start 155.5 47.63) (end 155.5 57.61) (width 0.2) (layer "F.Cu") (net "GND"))
 (segment (start 155.75 60.58) (end 155.75 70.06) (width 0.2) (layer "F.Cu") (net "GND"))
 (segment (start 135.2239 71.67) (end 136.36 71.67) (width 0.2) (layer "F.Cu") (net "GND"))
 (segment (start 137.7998 85.8098) (end 136.36 84.37) (width 0.2) (layer "F.Cu") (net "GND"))
 (segment (start 154.14 58.97) (end 155.75 60.58) (width 0.2) (layer "F.Cu") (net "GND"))
 (segment (start 134.25 61.08) (end 136.36 58.97) (width 0.2) (layer "F.Cu") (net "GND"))
 (segment (start 135 57.61) (end 135 47.63) (width 0.2) (layer "F.Cu") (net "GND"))
 (segment (start 151.725 79.725) (end 149.71 79.725) (width 0.2) (layer "F.Cu") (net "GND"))
 (via (at 151.75 79.75) (size 0.6) (drill 0.3) (layers "F.Cu" "B.Cu") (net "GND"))
 (segment (start 132.75 97.06) (end 136.87 97.06) (width 0.2) (layer "B.Cu") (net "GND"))
 (segment (start 136.36 46.27) (end 154.14 46.27) (width 0.2) (layer "B.Cu") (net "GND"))
 (segment (start 151.75 79.75) (end 151.75 74.06) (width 0.2) (layer "B.Cu") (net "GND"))
 (segment (start 136.87 97.06) (end 139.71 94.22) (width 0.2) (layer "B.Cu") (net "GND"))
 (segment (start 151.75 79.75) (end 151.75 81.98) (width 0.2) (layer "B.Cu") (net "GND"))
 (segment (start 151.75 74.06) (end 154.14 71.67) (width 0.2) (layer "B.Cu") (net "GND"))
 (segment (start 151.75 81.98) (end 154.14 84.37) (width 0.2) (layer "B.Cu") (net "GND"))
 (segment (start 144.745 82.25) (end 144.76 82.265) (width 0.2) (layer "F.Cu") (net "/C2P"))
 (segment (start 141.975 82.25) (end 144.745 82.25) (width 0.2) (layer "F.Cu") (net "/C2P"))
 (segment (start 141.5 82.725) (end 141.975 82.25) (width 0.2) (layer "F.Cu") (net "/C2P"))
 (segment (start 142.035 83.535) (end 144.76 83.535) (width 0.2) (layer "F.Cu") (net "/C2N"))
 (segment (start 142 83.5) (end 142.035 83.535) (width 0.2) (layer "F.Cu") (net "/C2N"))
 (segment (start 141.5 84) (end 142 83.5) (width 0.2) (layer "F.Cu") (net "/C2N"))
 (segment (start 141.5 84.275) (end 141.5 84) (width 0.2) (layer "F.Cu") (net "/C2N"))
 (segment (start 143.03 76.725) (end 144.76 78.455) (width 0.2) (layer "F.Cu") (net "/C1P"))
 (segment (start 141.5 76.725) (end 143.03 76.725) (width 0.2) (layer "F.Cu") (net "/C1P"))
 (segment (start 141.5 78.275) (end 144.22 80.995) (width 0.2) (layer "F.Cu") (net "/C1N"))
 (segment (start 144.22 80.995) (end 144.76 80.995) (width 0.2) (layer "F.Cu") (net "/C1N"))
 (segment (start 141.5 87.275) (end 143.97 84.805) (width 0.2) (layer "F.Cu") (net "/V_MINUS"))
 (segment (start 143.97 84.805) (end 144.76 84.805) (width 0.2) (layer "F.Cu") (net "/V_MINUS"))
 (segment (start 140.23 89.25) (end 138.75 87.77) (width 0.2) (layer "F.Cu") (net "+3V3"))
 (segment (start 148.3446 75.5946) (end 149.71 76.96) (width 0.2) (layer "F.Cu") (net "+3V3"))
 (segment (start 138.75 87.77) (end 138.75 76.2953) (width 0.2) (layer "F.Cu") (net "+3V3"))
 (segment (start 138 74.1439) (end 139.4507 75.5946) (width 0.2) (layer "F.Cu") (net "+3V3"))
 (segment (start 136.36 51.35) (end 138 52.99) (width 0.2) (layer "F.Cu") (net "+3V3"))
 (segment (start 138.75 76.2953) (end 139.4507 75.5946) (width 0.2) (layer "F.Cu") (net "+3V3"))
 (segment (start 138 52.99) (end 138 74.1439) (width 0.2) (layer "F.Cu") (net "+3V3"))
 (segment (start 149.71 76.96) (end 149.71 78.455) (width 0.2) (layer "F.Cu") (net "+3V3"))
 (segment (start 139.4507 75.5946) (end 148.3446 75.5946) (width 0.2) (layer "F.Cu") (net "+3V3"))
 (segment (start 150.0953 84.4197) (end 151.1935 84.4197) (width 0.2) (layer "F.Cu") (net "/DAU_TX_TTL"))
 (segment (start 149.71 84.805) (end 150.0953 84.4197) (width 0.2) (layer "F.Cu") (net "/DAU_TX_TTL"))
 (via (at 151.1935 84.4197) (size 0.6) (drill 0.3) (layers "F.Cu" "B.Cu") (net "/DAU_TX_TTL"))
 (segment (start 155.2548 77.8648) (end 155.2548 84.822) (width 0.2) (layer "B.Cu") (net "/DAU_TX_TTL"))
 (segment (start 155.2548 84.822) (end 154.5728 85.504) (width 0.2) (layer "B.Cu") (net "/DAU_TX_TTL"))
 (segment (start 152.2778 85.504) (end 151.1935 84.4197) (width 0.2) (layer "B.Cu") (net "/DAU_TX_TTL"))
 (segment (start 154.14 76.75) (end 155.2548 77.8648) (width 0.2) (layer "B.Cu") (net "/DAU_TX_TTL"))
 (segment (start 154.5728 85.504) (end 152.2778 85.504) (width 0.2) (layer "B.Cu") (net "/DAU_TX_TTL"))
 (segment (start 152.435 83.535) (end 149.71 83.535) (width 0.2) (layer "F.Cu") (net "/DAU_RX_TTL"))
 (segment (start 154.14 81.83) (end 152.435 83.535) (width 0.2) (layer "F.Cu") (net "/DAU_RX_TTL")))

